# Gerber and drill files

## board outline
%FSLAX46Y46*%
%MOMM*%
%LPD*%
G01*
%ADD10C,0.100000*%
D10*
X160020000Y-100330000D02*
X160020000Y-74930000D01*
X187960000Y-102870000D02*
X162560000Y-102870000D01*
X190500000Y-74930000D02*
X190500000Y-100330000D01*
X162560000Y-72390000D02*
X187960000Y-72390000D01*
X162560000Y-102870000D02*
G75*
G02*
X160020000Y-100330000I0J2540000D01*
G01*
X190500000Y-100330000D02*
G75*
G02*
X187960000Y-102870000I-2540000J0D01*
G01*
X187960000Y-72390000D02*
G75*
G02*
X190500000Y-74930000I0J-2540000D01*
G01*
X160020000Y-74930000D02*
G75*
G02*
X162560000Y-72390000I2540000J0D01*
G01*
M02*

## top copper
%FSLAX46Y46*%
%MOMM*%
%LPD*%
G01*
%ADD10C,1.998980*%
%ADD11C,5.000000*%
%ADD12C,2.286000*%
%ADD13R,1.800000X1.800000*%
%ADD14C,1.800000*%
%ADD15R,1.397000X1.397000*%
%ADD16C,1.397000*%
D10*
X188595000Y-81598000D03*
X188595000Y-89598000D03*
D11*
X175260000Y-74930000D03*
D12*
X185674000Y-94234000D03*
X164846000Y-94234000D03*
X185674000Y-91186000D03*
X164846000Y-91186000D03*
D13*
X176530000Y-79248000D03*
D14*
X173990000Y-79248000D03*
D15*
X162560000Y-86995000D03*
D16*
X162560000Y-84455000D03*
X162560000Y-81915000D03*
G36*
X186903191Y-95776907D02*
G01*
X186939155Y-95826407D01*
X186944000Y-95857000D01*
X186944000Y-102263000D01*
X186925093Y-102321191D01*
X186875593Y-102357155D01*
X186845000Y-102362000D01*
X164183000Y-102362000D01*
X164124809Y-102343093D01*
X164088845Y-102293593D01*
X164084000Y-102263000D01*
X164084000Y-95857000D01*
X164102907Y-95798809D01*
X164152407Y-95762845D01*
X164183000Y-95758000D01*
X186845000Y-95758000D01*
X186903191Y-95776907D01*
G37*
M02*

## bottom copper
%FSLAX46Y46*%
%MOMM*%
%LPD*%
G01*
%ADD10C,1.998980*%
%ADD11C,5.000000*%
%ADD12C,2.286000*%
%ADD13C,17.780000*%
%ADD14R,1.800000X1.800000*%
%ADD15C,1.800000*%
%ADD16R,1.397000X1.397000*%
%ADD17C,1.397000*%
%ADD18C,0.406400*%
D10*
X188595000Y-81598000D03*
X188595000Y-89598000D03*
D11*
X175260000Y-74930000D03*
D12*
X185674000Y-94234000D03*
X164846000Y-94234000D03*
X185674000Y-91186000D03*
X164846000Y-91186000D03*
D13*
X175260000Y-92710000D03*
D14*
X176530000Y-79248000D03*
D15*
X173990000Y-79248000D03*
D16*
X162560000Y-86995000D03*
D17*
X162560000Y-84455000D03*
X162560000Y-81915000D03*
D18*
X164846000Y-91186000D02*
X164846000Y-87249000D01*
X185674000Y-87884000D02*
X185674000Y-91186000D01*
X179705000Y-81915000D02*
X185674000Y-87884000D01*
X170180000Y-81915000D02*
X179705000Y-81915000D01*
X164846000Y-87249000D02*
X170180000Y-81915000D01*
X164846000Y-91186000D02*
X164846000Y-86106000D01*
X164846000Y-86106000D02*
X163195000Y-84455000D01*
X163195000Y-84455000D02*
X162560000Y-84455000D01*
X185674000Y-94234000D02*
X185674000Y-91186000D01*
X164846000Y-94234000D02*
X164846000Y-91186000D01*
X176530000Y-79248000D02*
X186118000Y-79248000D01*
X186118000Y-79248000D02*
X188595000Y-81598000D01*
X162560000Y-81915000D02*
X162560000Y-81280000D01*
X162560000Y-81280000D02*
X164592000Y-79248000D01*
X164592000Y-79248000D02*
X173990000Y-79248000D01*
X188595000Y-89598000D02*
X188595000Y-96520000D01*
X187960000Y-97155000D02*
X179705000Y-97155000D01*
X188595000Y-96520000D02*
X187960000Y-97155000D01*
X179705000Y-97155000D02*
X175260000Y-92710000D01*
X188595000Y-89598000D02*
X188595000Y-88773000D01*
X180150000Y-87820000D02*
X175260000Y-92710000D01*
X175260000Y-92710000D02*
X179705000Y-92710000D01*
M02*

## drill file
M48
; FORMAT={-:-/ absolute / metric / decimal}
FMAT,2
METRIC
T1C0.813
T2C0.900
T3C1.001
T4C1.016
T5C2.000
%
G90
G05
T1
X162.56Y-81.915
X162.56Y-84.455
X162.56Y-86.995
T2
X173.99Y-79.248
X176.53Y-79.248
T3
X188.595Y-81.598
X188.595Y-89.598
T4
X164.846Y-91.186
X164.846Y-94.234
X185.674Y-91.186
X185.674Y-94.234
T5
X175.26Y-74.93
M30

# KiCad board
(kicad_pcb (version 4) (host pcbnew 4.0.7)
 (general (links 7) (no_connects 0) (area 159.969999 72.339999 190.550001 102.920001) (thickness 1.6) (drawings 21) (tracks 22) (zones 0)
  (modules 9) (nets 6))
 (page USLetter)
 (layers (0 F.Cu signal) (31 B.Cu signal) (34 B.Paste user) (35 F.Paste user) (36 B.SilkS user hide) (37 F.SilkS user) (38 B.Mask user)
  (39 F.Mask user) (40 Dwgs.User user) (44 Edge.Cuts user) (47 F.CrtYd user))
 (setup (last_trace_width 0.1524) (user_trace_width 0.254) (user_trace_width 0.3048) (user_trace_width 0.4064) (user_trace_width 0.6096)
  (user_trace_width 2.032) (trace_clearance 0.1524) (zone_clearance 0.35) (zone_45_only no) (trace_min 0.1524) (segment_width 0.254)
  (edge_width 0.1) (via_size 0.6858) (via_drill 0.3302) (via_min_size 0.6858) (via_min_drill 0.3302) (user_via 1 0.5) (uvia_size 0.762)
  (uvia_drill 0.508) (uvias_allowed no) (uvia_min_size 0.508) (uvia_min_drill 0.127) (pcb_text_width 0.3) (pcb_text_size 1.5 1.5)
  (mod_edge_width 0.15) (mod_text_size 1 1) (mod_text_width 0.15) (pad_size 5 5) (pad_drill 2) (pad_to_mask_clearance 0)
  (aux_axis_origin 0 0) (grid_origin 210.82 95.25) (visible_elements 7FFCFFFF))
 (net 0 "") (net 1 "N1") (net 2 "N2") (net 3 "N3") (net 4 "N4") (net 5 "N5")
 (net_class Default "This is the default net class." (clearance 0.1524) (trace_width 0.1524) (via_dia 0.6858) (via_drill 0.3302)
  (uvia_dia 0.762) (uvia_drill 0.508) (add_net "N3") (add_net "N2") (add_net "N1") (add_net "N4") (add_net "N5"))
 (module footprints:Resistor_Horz (layer F.Cu) (at 188.595 85.598 270)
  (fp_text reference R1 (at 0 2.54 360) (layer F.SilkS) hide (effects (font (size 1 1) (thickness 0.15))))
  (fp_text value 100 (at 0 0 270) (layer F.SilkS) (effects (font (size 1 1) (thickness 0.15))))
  (pad 1 thru_hole circle (at -4 0 270) (size 1.99898 1.99898) (drill 1.00076) (layers *.Cu *.SilkS *.Mask) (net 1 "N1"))
  (pad 2 thru_hole circle (at 4 0 270) (size 1.99898 1.99898) (drill 1.00076) (layers *.Cu *.SilkS *.Mask) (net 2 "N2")))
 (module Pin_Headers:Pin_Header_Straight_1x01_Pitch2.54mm (layer F.Cu) (at 175.26 74.93)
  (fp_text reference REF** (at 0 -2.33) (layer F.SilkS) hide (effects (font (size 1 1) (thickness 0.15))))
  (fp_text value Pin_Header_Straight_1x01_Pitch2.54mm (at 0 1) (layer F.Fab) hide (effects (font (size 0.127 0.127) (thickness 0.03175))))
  (pad 1 thru_hole circle (at 0 0) (size 5 5) (drill 2) (layers *.Cu B.Mask)))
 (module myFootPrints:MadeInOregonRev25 (layer F.Cu) (at 167.64 76.454)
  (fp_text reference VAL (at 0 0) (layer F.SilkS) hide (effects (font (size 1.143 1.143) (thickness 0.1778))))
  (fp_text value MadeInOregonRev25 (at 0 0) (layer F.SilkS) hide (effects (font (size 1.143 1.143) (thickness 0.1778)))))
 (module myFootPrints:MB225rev (layer F.Cu) (at 184.15 76.2)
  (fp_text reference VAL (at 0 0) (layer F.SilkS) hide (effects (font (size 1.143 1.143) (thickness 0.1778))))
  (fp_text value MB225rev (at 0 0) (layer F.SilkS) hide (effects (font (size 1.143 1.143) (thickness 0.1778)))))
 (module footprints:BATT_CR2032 (layer B.Cu) (at 175.26 92.71 180)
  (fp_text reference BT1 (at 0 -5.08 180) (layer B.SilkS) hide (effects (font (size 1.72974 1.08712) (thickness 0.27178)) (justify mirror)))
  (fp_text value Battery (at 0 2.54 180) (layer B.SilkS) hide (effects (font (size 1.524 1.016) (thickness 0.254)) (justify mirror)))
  (pad 1 thru_hole circle (at -10.414 -1.524 180) (size 2.286 2.286) (drill 1.016) (layers *.Cu *.Mask B.SilkS) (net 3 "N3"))
  (pad 1 thru_hole circle (at 10.414 -1.524 180) (size 2.286 2.286) (drill 1.016) (layers *.Cu *.Mask B.SilkS) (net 3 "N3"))
  (pad 1 thru_hole circle (at -10.414 1.524 180) (size 2.286 2.286) (drill 1.016) (layers *.Cu *.Mask B.SilkS) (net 3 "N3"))
  (pad 1 thru_hole circle (at 10.414 1.524 180) (size 2.286 2.286) (drill 1.016) (layers *.Cu *.Mask B.SilkS) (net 3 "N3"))
  (pad 2 smd circle (at 0 0 180) (size 17.78 17.78) (layers B.Cu B.Paste B.Mask) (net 2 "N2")))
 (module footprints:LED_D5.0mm (layer F.Cu) (at 176.53 79.248 180)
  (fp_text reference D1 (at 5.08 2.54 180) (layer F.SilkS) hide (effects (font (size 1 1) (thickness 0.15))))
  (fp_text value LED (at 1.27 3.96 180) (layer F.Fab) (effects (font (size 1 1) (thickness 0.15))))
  (pad 1 thru_hole rect (at 0 0 180) (size 1.8 1.8) (drill 0.9) (layers *.Cu *.Mask) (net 1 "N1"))
  (pad 2 thru_hole circle (at 2.54 0 180) (size 1.8 1.8) (drill 0.9) (layers *.Cu *.Mask) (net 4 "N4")))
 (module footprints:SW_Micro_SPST (layer F.Cu) (at 162.56 84.455 90)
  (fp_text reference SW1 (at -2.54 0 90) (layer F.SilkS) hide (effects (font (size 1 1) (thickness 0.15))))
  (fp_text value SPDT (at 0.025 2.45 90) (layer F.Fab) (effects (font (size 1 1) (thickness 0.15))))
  (pad 1 thru_hole rect (at -2.54 0 90) (size 1.397 1.397) (drill 0.8128) (layers *.Cu *.Mask F.SilkS) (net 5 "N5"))
  (pad 2 thru_hole circle (at 0 0 90) (size 1.397 1.397) (drill 0.8128) (layers *.Cu *.Mask F.SilkS) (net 3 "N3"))
  (pad 3 thru_hole circle (at 2.54 0 90) (size 1.397 1.397) (drill 0.8128) (layers *.Cu *.Mask F.SilkS) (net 4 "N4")))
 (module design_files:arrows (layer F.Cu) (at 179.07 77.47)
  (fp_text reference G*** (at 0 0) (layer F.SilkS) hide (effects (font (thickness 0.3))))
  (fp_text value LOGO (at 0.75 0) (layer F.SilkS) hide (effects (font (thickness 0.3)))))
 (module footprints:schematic (layer F.Cu) (at 175.26 87.503)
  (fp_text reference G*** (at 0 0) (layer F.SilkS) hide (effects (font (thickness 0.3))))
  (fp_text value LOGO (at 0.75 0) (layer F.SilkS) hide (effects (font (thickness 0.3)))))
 (gr_line (start 160.02 100.33) (end 160.02 74.93) (angle 90) (layer Edge.Cuts) (width 0.1))
 (gr_line (start 187.96 102.87) (end 162.56 102.87) (angle 90) (layer Edge.Cuts) (width 0.1))
 (gr_line (start 190.5 74.93) (end 190.5 100.33) (angle 90) (layer Edge.Cuts) (width 0.1))
 (gr_line (start 162.56 72.39) (end 187.96 72.39) (angle 90) (layer Edge.Cuts) (width 0.1))
 (gr_arc (start 162.56 100.33) (end 162.56 102.87) (angle 90) (layer Edge.Cuts) (width 0.1))
 (gr_arc (start 187.96 100.33) (end 190.5 100.33) (angle 90) (layer Edge.Cuts) (width 0.1))
 (gr_arc (start 187.96 74.93) (end 187.96 72.39) (angle 90) (layer Edge.Cuts) (width 0.1))
 (gr_arc (start 162.56 74.93) (end 160.02 74.93) (angle 90) (layer Edge.Cuts) (width 0.1))
 (segment (start 164.846 91.186) (end 164.846 87.249) (width 0.4064) (layer B.Cu) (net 3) (status 10))
 (segment (start 185.674 87.884) (end 185.674 91.186) (width 0.4064) (layer B.Cu) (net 3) (status 20))
 (segment (start 179.705 81.915) (end 185.674 87.884) (width 0.4064) (layer B.Cu) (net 3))
 (segment (start 170.18 81.915) (end 179.705 81.915) (width 0.4064) (layer B.Cu) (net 3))
 (segment (start 164.846 87.249) (end 170.18 81.915) (width 0.4064) (layer B.Cu) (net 3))
 (segment (start 164.846 91.186) (end 164.846 86.106) (width 0.4064) (layer B.Cu) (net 3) (status 10))
 (segment (start 164.846 86.106) (end 163.195 84.455) (width 0.4064) (layer B.Cu) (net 3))
 (segment (start 163.195 84.455) (end 162.56 84.455) (width 0.4064) (layer B.Cu) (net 3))
 (segment (start 185.674 94.234) (end 185.674 91.186) (width 0.4064) (layer B.Cu) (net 3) (status 30))
 (segment (start 164.846 94.234) (end 164.846 91.186) (width 0.4064) (layer B.Cu) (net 3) (status 30))
 (segment (start 176.53 79.248) (end 186.118 79.248) (width 0.4064) (layer B.Cu) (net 1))
 (segment (start 186.118 79.248) (end 188.595 81.598) (width 0.4064) (layer B.Cu) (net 1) (status 20))
 (segment (start 162.56 81.915) (end 162.56 81.28) (width 0.4064) (layer B.Cu) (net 4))
 (segment (start 162.56 81.28) (end 164.592 79.248) (width 0.4064) (layer B.Cu) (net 4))
 (segment (start 164.592 79.248) (end 173.99 79.248) (width 0.4064) (layer B.Cu) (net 4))
 (segment (start 188.595 89.598) (end 188.595 96.52) (width 0.4064) (layer B.Cu) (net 2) (status 10))
 (segment (start 187.96 97.155) (end 179.705 97.155) (width 0.4064) (layer B.Cu) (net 2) (status 20))
 (segment (start 188.595 96.52) (end 187.96 97.155) (width 0.4064) (layer B.Cu) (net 2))
 (segment (start 179.705 97.155) (end 175.26 92.71) (width 0.4064) (layer B.Cu) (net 2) (status 30))
 (segment (start 188.595 89.598) (end 188.595 88.773) (width 0.4064) (layer B.Cu) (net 2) (status 30))
 (segment (start 180.15 87.82) (end 175.26 92.71) (width 0.4064) (layer B.Cu) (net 2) (status 30))
 (segment (start 175.26 92.71) (end 179.705 92.71) (width 0.4064) (layer B.Cu) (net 2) (status 30))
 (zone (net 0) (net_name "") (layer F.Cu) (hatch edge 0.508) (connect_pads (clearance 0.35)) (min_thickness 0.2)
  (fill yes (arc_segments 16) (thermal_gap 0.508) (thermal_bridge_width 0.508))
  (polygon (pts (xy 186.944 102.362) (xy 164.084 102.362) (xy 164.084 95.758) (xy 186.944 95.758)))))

